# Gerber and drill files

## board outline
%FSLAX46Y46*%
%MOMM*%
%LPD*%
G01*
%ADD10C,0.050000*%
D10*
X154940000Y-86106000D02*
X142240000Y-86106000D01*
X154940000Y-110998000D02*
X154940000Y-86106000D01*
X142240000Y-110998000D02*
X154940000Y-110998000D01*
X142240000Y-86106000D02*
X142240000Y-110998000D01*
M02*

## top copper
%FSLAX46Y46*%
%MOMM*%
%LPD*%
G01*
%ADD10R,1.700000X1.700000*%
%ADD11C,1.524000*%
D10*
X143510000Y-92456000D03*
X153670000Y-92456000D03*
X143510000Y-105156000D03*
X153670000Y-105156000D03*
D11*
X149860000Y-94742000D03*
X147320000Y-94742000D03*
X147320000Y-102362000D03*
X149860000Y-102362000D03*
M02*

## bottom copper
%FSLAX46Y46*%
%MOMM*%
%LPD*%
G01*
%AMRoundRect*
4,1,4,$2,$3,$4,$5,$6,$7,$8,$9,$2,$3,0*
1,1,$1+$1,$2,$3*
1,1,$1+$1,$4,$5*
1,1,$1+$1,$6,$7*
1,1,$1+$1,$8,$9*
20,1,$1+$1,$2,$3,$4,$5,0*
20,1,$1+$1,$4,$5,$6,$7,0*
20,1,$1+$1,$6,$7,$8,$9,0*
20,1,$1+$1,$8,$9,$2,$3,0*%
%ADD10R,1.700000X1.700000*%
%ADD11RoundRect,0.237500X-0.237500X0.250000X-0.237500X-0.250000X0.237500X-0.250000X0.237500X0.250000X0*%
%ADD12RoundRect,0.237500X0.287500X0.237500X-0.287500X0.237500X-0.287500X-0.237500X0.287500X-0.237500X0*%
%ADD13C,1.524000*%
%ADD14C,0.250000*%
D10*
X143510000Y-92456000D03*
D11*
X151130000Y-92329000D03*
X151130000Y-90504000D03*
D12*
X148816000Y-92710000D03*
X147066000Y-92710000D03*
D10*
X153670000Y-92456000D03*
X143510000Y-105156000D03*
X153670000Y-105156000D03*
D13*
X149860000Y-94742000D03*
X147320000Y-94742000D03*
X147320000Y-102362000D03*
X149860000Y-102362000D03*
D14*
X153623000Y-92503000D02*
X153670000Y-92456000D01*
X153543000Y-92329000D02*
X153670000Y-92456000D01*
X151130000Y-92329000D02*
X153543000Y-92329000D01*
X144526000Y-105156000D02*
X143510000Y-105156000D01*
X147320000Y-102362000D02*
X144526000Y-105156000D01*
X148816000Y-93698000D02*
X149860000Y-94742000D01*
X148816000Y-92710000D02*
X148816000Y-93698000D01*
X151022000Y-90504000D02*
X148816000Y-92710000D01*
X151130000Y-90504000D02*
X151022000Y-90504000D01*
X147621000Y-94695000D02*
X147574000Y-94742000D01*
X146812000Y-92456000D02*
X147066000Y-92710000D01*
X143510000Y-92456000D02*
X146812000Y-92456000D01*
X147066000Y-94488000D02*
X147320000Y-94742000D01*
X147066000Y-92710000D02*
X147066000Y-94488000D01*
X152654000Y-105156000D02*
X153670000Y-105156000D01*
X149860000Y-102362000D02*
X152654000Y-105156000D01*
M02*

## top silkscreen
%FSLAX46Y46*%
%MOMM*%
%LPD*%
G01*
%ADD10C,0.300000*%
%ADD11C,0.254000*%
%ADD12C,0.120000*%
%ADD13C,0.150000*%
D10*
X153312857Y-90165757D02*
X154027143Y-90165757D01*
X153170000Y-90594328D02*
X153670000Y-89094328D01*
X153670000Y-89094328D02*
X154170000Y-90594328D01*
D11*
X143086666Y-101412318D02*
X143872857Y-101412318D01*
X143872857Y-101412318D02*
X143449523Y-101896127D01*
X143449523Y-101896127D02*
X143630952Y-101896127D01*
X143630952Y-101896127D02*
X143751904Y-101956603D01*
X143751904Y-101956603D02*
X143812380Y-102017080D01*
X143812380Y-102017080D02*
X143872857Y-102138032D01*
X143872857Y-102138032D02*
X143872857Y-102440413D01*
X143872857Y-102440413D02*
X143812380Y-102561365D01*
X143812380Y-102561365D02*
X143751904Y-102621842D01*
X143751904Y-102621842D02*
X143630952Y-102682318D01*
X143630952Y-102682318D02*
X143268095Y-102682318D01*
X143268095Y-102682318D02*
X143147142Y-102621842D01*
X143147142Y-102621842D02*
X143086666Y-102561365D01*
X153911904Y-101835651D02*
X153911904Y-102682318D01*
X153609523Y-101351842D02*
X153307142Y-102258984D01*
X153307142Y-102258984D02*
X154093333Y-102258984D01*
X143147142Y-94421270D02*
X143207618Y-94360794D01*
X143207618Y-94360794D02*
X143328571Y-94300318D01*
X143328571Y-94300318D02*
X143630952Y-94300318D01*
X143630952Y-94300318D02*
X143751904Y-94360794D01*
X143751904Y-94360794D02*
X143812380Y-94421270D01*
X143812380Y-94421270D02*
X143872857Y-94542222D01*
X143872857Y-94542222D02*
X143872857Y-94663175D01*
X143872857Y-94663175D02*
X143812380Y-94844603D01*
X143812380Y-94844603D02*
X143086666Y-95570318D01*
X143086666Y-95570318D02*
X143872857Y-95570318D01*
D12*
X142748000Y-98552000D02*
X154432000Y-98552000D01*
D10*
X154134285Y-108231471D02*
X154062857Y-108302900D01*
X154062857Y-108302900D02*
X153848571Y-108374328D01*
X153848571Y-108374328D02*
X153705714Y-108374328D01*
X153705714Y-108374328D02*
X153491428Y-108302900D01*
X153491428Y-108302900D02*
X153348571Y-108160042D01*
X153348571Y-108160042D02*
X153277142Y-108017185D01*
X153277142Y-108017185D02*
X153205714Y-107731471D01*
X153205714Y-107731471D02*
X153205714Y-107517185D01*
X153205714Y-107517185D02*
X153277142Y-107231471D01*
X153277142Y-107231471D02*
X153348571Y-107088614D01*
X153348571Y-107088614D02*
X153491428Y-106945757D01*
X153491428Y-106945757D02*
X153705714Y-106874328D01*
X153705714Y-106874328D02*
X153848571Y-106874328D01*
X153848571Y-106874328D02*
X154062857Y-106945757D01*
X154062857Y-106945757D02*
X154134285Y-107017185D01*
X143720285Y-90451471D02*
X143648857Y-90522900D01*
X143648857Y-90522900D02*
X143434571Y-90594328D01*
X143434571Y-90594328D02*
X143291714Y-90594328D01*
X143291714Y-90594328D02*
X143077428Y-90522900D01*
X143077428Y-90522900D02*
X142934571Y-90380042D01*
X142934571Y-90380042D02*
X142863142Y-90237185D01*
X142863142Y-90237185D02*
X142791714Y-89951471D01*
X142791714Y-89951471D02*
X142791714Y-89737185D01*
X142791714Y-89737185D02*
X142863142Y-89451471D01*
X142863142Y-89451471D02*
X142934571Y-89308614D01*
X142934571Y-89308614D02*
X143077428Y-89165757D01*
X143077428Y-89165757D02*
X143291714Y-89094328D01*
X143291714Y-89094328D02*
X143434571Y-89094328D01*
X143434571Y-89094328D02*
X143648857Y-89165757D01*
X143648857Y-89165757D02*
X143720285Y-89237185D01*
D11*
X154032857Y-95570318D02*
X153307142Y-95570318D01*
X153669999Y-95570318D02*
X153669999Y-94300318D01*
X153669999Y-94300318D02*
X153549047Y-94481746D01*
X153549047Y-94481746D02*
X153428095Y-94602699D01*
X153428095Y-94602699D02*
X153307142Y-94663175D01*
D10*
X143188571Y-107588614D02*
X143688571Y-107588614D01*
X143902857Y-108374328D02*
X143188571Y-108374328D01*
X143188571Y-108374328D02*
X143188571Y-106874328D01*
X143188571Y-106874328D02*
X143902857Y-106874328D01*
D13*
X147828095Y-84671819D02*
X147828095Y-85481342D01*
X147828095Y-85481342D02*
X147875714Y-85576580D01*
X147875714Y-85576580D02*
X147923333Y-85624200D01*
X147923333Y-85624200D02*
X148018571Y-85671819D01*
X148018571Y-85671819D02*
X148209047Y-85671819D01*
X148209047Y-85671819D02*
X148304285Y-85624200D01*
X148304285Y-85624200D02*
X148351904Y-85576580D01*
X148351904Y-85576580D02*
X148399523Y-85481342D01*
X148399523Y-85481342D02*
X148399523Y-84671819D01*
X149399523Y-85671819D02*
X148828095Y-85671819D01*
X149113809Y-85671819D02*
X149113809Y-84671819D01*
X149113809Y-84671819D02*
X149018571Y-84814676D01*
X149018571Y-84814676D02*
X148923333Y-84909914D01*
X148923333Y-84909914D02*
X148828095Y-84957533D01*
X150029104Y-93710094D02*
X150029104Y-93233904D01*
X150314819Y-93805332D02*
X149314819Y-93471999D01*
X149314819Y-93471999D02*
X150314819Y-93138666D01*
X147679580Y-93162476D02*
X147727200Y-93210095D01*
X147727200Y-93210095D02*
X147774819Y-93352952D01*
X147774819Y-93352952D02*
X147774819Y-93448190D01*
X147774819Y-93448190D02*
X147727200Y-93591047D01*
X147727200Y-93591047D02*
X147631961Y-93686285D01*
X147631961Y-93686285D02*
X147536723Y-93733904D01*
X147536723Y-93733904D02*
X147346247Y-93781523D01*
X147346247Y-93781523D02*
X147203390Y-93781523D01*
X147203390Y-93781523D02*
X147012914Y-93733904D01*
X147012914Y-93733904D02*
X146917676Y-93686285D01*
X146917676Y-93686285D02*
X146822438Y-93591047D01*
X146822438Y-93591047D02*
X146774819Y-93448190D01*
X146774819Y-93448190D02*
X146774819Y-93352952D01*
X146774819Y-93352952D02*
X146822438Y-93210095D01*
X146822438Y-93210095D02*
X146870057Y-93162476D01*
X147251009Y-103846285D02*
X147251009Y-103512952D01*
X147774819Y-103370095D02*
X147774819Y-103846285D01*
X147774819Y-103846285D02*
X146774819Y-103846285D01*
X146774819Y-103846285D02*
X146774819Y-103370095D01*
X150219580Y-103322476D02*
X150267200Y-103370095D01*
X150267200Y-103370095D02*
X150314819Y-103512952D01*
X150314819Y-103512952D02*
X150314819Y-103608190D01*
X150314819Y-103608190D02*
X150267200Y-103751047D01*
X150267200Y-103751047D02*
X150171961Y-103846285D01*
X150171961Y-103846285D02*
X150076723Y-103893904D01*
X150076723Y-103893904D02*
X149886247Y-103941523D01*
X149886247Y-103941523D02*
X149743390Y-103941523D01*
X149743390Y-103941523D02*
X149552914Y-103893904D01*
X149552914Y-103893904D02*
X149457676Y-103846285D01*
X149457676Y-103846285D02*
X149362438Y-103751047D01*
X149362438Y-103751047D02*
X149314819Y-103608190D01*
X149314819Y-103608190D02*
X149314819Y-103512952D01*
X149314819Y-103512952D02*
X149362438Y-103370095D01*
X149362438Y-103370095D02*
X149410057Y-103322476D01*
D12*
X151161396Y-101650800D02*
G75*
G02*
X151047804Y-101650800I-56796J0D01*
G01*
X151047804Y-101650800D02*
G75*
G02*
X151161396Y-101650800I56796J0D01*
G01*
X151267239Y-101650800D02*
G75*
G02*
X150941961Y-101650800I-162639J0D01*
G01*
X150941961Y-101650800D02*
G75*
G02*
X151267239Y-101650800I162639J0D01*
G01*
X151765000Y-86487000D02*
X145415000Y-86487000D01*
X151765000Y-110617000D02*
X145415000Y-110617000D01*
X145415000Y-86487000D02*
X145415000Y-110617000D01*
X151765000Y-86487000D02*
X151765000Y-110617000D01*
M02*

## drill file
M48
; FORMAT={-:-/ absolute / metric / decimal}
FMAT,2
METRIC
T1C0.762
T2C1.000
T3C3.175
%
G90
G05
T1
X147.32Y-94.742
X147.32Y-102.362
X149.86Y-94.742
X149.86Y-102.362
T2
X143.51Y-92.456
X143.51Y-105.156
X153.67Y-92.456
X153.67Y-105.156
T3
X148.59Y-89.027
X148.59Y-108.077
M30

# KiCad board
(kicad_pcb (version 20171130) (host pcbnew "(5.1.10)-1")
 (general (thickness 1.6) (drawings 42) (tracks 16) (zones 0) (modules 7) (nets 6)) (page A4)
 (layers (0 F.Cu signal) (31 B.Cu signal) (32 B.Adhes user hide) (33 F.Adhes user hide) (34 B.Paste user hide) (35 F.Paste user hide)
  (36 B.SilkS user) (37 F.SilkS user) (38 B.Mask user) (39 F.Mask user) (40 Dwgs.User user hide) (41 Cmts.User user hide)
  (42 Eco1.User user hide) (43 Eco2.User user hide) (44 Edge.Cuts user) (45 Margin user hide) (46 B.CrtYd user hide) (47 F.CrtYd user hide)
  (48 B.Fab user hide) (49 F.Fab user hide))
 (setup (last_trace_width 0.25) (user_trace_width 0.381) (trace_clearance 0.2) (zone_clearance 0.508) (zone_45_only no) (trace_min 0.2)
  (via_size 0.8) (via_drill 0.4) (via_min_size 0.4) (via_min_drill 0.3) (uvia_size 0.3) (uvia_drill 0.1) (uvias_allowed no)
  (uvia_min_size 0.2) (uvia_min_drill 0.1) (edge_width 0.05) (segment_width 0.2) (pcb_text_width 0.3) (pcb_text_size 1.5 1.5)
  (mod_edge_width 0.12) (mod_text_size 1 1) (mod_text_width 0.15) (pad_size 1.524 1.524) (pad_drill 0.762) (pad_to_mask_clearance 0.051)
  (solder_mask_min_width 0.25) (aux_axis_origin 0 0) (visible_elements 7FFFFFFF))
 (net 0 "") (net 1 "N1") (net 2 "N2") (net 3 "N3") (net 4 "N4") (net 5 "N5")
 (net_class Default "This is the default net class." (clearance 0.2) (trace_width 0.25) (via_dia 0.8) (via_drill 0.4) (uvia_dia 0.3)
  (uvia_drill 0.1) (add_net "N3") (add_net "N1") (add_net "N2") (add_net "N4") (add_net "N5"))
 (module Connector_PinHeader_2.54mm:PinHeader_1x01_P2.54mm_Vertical (layer B.Cu) (at 143.51 92.456 180)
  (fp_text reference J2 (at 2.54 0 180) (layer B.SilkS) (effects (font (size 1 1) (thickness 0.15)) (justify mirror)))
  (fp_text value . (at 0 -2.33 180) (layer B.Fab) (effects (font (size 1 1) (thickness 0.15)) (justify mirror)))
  (pad 1 thru_hole rect (at 0 0 180) (size 1.7 1.7) (drill 1) (layers *.Cu *.Mask) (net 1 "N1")))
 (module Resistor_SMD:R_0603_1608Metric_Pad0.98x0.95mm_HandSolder (layer B.Cu) (at 151.13 91.4165 270)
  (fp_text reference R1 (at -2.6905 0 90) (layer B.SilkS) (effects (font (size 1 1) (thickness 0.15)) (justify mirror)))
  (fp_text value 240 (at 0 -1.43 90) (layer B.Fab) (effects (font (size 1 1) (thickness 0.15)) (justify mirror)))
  (pad 2 smd roundrect (at 0.9125 0 270) (size 0.975 0.95) (layers B.Cu B.Paste B.Mask) (roundrect_rratio 0.25) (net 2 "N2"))
  (pad 1 smd roundrect (at -0.9125 0 270) (size 0.975 0.95) (layers B.Cu B.Paste B.Mask) (roundrect_rratio 0.25) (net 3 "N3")))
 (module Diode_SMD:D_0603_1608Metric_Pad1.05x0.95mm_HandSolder (layer B.Cu) (at 147.941 92.71 180)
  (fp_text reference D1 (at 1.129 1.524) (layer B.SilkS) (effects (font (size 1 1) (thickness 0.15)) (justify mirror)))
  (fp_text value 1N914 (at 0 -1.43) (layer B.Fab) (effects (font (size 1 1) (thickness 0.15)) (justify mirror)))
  (pad 1 smd roundrect (at -0.875 0 180) (size 1.05 0.95) (layers B.Cu B.Paste B.Mask) (roundrect_rratio 0.25) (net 3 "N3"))
  (pad 2 smd roundrect (at 0.875 0 180) (size 1.05 0.95) (layers B.Cu B.Paste B.Mask) (roundrect_rratio 0.25) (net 1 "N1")))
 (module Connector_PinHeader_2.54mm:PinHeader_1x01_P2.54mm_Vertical (layer B.Cu) (at 153.67 92.456 180)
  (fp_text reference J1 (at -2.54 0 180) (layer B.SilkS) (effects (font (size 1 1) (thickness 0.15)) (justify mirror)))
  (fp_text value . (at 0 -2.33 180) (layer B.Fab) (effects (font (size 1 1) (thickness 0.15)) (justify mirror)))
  (pad 1 thru_hole rect (at 0 0 180) (size 1.7 1.7) (drill 1) (layers *.Cu *.Mask) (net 2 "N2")))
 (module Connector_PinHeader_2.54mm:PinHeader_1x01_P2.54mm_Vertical (layer B.Cu) (at 143.51 105.156 180)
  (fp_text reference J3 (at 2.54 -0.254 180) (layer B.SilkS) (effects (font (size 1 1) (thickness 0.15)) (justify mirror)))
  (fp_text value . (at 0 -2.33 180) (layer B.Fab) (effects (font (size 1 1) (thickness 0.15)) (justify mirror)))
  (pad 1 thru_hole rect (at 0 0 180) (size 1.7 1.7) (drill 1) (layers *.Cu *.Mask) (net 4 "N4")))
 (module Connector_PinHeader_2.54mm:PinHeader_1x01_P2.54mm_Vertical (layer B.Cu) (at 153.67 105.156 180)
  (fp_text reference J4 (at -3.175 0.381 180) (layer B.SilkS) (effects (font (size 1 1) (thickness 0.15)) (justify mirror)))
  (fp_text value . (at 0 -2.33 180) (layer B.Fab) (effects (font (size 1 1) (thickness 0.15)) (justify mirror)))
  (pad 1 thru_hole rect (at 0 0 180) (size 1.7 1.7) (drill 1) (layers *.Cu *.Mask) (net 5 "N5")))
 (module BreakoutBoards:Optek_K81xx (layer F.Cu) (at 148.59 98.552 90)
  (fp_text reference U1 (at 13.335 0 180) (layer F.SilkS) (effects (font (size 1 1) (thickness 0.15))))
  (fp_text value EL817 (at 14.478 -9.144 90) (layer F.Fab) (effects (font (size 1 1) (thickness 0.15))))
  (fp_circle (center -3.0988 2.5146) (end -3.1496 2.4892) (layer F.SilkS) (width 0.12))
  (fp_circle (center -3.0988 2.5146) (end -3.2004 2.3876) (layer F.SilkS) (width 0.12))
  (fp_line (start 12.065 3.175) (end 12.065 -3.175) (layer F.SilkS) (width 0.12))
  (fp_line (start -12.065 3.175) (end -12.065 -3.175) (layer F.SilkS) (width 0.12))
  (fp_line (start 12.065 -3.175) (end -12.065 -3.175) (layer F.SilkS) (width 0.12))
  (fp_line (start 12.065 3.175) (end -12.065 3.175) (layer F.SilkS) (width 0.12))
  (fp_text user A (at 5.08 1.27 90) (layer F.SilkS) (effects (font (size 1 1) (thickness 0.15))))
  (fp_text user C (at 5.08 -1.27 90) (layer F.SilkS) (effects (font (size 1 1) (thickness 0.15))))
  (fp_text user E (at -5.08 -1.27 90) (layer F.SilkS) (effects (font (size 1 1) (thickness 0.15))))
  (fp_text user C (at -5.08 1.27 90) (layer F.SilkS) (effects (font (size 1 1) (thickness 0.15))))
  (pad 1 thru_hole circle (at 3.81 1.27) (size 1.524 1.524) (drill 0.762) (layers *.Cu *.Mask) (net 3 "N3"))
  (pad 2 thru_hole circle (at 3.81 -1.27) (size 1.524 1.524) (drill 0.762) (layers *.Cu *.Mask) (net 1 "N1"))
  (pad 3 thru_hole circle (at -3.81 -1.27) (size 1.524 1.524) (drill 0.762) (layers *.Cu *.Mask) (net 4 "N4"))
  (pad 4 thru_hole circle (at -3.81 1.27) (size 1.524 1.524) (drill 0.762) (layers *.Cu *.Mask) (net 5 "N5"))
  (pad "" np_thru_hole circle (at 9.525 0) (size 3.175 3.175) (drill 3.175) (layers *.Cu *.Mask))
  (pad "" np_thru_hole circle (at -9.525 0) (size 3.175 3.175) (drill 3.175) (layers *.Cu *.Mask)))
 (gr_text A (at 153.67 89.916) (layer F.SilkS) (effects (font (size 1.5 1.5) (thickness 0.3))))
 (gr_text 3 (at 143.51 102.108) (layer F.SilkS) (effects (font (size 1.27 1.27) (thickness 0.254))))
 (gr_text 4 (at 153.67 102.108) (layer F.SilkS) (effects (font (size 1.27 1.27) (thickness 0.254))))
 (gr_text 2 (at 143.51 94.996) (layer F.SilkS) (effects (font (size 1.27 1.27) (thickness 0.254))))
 (gr_line (start 142.748 98.552) (end 154.432 98.552) (layer F.SilkS) (width 0.12))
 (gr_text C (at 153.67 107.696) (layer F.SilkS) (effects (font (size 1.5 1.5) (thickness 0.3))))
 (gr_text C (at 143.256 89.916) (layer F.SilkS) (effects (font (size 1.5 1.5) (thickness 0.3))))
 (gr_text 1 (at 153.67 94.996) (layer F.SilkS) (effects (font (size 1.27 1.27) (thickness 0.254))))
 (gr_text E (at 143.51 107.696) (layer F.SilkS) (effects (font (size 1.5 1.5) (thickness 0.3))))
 (gr_line (start 154.94 86.106) (end 142.24 86.106) (layer Edge.Cuts) (width 0.05))
 (gr_line (start 154.94 110.998) (end 154.94 86.106) (layer Edge.Cuts) (width 0.05))
 (gr_line (start 142.24 110.998) (end 154.94 110.998) (layer Edge.Cuts) (width 0.05))
 (gr_line (start 142.24 86.106) (end 142.24 110.998) (layer Edge.Cuts) (width 0.05))
 (segment (start 153.623 92.503) (end 153.67 92.456) (width 0.25) (layer B.Cu) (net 2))
 (segment (start 153.543 92.329) (end 153.67 92.456) (width 0.25) (layer B.Cu) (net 2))
 (segment (start 151.13 92.329) (end 153.543 92.329) (width 0.25) (layer B.Cu) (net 2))
 (segment (start 144.526 105.156) (end 143.51 105.156) (width 0.25) (layer B.Cu) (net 4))
 (segment (start 147.32 102.362) (end 144.526 105.156) (width 0.25) (layer B.Cu) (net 4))
 (segment (start 148.816 93.698) (end 149.86 94.742) (width 0.25) (layer B.Cu) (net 3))
 (segment (start 148.816 92.71) (end 148.816 93.698) (width 0.25) (layer B.Cu) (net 3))
 (segment (start 151.022 90.504) (end 148.816 92.71) (width 0.25) (layer B.Cu) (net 3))
 (segment (start 151.13 90.504) (end 151.022 90.504) (width 0.25) (layer B.Cu) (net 3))
 (segment (start 147.621 94.695) (end 147.574 94.742) (width 0.25) (layer B.Cu) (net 1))
 (segment (start 146.812 92.456) (end 147.066 92.71) (width 0.25) (layer B.Cu) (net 1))
 (segment (start 143.51 92.456) (end 146.812 92.456) (width 0.25) (layer B.Cu) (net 1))
 (segment (start 147.066 94.488) (end 147.32 94.742) (width 0.25) (layer B.Cu) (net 1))
 (segment (start 147.066 92.71) (end 147.066 94.488) (width 0.25) (layer B.Cu) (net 1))
 (segment (start 152.654 105.156) (end 153.67 105.156) (width 0.25) (layer B.Cu) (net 5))
 (segment (start 149.86 102.362) (end 152.654 105.156) (width 0.25) (layer B.Cu) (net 5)))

